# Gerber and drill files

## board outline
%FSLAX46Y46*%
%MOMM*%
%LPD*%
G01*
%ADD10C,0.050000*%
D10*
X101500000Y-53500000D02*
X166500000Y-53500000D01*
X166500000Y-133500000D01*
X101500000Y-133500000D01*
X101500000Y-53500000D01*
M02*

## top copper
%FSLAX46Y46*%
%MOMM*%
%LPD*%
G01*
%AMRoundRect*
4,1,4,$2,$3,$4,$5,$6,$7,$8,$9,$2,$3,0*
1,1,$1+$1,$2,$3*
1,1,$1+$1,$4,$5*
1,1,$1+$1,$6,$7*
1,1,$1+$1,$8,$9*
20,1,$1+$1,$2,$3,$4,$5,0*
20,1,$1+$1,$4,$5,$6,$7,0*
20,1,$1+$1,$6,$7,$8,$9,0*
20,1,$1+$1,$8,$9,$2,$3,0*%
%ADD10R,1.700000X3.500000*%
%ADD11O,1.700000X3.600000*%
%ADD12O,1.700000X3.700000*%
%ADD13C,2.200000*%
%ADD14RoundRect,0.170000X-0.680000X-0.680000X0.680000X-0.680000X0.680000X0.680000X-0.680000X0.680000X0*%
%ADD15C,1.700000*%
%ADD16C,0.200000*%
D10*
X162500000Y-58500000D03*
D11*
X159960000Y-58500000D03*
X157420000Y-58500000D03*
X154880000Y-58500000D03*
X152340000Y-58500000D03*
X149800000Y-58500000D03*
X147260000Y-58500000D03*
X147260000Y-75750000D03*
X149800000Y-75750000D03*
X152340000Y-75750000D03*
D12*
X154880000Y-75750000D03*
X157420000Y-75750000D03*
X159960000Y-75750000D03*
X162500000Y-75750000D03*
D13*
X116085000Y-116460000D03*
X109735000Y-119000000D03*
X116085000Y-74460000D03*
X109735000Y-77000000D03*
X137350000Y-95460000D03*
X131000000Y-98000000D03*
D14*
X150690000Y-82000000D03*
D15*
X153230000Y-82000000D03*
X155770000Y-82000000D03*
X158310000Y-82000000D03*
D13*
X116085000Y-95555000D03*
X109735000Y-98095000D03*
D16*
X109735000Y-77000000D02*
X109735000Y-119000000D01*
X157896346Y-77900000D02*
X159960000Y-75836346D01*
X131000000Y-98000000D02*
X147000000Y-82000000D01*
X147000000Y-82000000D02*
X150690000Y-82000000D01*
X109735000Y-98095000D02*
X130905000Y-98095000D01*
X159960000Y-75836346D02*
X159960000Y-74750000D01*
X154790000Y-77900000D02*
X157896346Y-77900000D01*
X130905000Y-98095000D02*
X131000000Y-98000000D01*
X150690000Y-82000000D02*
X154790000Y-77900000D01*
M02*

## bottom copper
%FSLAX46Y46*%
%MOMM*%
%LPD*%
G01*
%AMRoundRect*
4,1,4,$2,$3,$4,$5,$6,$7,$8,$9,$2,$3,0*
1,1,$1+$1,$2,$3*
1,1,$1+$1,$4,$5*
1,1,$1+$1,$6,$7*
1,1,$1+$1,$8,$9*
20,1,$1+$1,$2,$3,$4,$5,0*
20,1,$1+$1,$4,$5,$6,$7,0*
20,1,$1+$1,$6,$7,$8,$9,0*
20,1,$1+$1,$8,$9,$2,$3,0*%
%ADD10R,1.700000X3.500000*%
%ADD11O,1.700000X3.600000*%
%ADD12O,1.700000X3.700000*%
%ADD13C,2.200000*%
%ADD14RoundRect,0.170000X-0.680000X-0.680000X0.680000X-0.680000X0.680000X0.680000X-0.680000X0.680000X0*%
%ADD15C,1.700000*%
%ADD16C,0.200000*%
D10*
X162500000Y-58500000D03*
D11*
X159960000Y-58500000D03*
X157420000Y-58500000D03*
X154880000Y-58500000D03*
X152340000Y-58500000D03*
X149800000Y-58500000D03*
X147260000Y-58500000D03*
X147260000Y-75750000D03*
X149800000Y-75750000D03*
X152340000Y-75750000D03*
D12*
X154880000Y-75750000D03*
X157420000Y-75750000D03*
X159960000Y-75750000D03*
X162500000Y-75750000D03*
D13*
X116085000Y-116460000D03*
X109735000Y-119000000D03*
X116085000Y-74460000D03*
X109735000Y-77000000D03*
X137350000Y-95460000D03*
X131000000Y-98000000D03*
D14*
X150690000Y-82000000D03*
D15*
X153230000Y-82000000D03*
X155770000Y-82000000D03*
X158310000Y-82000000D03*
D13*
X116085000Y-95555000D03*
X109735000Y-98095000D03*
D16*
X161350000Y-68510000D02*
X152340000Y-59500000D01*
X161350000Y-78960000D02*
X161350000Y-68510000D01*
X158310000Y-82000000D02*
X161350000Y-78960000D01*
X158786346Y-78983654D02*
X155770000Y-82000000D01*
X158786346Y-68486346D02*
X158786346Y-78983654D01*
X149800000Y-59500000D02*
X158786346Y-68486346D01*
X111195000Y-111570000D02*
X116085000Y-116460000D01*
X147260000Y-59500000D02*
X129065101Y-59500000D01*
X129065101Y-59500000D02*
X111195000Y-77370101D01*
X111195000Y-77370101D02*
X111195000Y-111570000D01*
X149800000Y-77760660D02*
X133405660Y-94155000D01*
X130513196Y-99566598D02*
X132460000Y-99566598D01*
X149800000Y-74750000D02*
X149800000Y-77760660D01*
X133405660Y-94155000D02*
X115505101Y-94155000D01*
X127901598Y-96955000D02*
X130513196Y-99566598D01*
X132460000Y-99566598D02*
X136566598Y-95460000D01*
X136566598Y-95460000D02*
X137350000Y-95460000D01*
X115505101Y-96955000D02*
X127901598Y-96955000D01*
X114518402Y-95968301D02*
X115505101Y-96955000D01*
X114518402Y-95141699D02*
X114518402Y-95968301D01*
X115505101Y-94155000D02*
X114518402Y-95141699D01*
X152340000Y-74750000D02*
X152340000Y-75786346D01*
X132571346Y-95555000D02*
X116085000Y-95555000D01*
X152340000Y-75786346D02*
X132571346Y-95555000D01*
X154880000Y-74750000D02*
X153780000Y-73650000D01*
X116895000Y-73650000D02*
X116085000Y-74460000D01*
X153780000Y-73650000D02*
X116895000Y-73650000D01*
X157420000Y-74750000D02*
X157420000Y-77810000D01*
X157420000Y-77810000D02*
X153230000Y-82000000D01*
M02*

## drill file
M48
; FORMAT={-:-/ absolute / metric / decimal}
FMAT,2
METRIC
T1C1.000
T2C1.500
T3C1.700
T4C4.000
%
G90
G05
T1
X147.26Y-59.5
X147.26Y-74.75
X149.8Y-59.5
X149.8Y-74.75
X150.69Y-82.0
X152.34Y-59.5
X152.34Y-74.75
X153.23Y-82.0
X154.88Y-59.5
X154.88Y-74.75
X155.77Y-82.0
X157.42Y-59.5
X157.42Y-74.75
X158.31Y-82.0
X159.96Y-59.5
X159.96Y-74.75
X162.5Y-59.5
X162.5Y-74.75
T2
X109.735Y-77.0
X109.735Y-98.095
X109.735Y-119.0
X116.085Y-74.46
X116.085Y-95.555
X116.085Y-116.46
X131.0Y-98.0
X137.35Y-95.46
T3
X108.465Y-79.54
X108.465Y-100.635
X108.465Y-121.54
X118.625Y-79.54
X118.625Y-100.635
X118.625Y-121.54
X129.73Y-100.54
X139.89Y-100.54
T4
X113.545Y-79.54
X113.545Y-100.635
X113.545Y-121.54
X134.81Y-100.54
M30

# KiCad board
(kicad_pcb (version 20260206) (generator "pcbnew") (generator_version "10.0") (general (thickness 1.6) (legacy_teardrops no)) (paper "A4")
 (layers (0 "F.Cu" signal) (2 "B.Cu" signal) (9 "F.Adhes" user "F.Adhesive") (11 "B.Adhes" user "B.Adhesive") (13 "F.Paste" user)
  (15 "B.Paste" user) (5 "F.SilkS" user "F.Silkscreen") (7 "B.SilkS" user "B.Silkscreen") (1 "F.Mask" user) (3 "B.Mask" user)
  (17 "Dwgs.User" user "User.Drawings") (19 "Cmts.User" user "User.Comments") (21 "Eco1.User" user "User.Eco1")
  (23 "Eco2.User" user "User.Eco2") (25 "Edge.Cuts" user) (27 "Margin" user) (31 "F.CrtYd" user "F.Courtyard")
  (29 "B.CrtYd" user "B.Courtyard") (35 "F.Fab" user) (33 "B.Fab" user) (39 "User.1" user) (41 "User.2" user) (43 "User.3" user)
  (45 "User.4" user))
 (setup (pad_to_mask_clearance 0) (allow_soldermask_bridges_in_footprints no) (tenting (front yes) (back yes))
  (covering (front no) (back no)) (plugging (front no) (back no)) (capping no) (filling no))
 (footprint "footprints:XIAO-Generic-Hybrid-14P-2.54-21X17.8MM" (layer "F.Cu") (at 154.88 67.125 -90)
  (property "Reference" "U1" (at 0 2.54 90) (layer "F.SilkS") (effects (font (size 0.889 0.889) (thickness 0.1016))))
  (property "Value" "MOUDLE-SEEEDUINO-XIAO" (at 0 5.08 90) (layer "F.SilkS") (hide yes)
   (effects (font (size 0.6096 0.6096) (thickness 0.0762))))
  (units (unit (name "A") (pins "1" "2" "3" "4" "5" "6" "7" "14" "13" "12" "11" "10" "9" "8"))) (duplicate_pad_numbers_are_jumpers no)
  (pad "1" thru_hole rect (at -7.625 -7.62 270) (size 3.5 1.7) (drill 1 (offset -1 0)) (layers "*.Cu" "*.Mask") (remove_unused_layers no)
   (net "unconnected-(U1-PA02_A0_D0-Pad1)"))
  (pad "2" thru_hole oval (at -7.625 -5.08 270) (size 3.6 1.7) (drill 1 (offset -1 0)) (layers "*.Cu" "*.Mask") (remove_unused_layers no)
   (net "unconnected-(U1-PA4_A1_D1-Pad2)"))
  (pad "3" thru_hole oval (at -7.625 -2.54 270) (size 3.6 1.7) (drill 1 (offset -1 0)) (layers "*.Cu" "*.Mask") (remove_unused_layers no)
   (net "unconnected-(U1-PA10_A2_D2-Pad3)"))
  (pad "4" thru_hole oval (at -7.625 0 270) (size 3.6 1.7) (drill 1 (offset -1 0)) (layers "*.Cu" "*.Mask") (remove_unused_layers no)
   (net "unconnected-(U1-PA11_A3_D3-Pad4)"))
  (pad "5" thru_hole oval (at -7.625 2.54 270) (size 3.6 1.7) (drill 1 (offset -1 0)) (layers "*.Cu" "*.Mask") (remove_unused_layers no)
   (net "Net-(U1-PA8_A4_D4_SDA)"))
  (pad "6" thru_hole oval (at -7.625 5.08 90) (size 3.6 1.7) (drill 1 (offset 1 0)) (layers "*.Cu" "*.Mask") (remove_unused_layers no)
   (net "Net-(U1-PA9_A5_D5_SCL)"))
  (pad "7" thru_hole oval (at -7.625 7.62 270) (size 3.6 1.7) (drill 1 (offset -1 0)) (layers "*.Cu" "*.Mask") (remove_unused_layers no)
   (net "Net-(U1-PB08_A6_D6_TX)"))
  (pad "8" thru_hole oval (at 7.625 7.62 270) (size 3.6 1.7) (drill 1 (offset 1 0)) (layers "*.Cu" "*.Mask") (remove_unused_layers no)
   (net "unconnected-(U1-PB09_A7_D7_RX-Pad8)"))
  (pad "9" thru_hole oval (at 7.625 5.08 270) (size 3.6 1.7) (drill 1 (offset 1 0)) (layers "*.Cu" "*.Mask") (remove_unused_layers no)
   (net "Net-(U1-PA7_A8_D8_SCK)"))
  (pad "10" thru_hole oval (at 7.625 2.54 270) (size 3.6 1.7) (drill 1 (offset 1 0)) (layers "*.Cu" "*.Mask") (remove_unused_layers no)
   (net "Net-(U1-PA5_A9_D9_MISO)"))
  (pad "11" thru_hole oval (at 7.625 0 270) (size 3.7 1.7) (drill 1 (offset 1 0)) (layers "*.Cu" "*.Mask") (remove_unused_layers no)
   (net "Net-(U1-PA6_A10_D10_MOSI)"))
  (pad "12" thru_hole oval (at 7.625 -2.54 270) (size 3.7 1.7) (drill 1 (offset 1 0)) (layers "*.Cu" "*.Mask") (remove_unused_layers no)
   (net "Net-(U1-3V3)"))
  (pad "13" thru_hole oval (at 7.625 -5.08 270) (size 3.7 1.7) (drill 1 (offset 1 0)) (layers "*.Cu" "*.Mask") (remove_unused_layers no)
   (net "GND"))
  (pad "14" thru_hole oval (at 7.625 -7.62 270) (size 3.7 1.7) (drill 1 (offset 1 0)) (layers "*.Cu" "*.Mask") (remove_unused_layers no)
   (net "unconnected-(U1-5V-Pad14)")))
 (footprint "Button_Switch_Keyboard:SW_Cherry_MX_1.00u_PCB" (layer "F.Cu") (at 116.085 116.46)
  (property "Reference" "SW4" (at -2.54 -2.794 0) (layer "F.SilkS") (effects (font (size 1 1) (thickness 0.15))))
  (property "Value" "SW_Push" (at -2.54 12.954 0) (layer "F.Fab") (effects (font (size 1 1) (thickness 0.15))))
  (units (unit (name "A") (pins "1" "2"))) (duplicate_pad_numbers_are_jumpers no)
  (pad "" np_thru_hole circle (at -7.62 5.08) (size 1.7 1.7) (drill 1.7) (layers "*.Cu" "*.Mask"))
  (pad "" np_thru_hole circle (at -2.54 5.08) (size 4 4) (drill 4) (layers "*.Cu" "*.Mask"))
  (pad "" np_thru_hole circle (at 2.54 5.08) (size 1.7 1.7) (drill 1.7) (layers "*.Cu" "*.Mask"))
  (pad "1" thru_hole circle (at 0 0) (size 2.2 2.2) (drill 1.5) (layers "*.Cu" "*.Mask") (remove_unused_layers no)
   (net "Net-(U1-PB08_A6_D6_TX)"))
  (pad "2" thru_hole circle (at -6.35 2.54) (size 2.2 2.2) (drill 1.5) (layers "*.Cu" "*.Mask") (remove_unused_layers no) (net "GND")))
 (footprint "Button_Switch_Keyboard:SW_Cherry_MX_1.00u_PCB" (layer "F.Cu") (at 116.085 74.46)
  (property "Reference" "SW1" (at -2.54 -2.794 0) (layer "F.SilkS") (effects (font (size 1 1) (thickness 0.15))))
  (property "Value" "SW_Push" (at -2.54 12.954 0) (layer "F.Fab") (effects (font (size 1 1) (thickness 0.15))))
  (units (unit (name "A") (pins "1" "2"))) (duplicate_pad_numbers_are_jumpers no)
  (pad "" np_thru_hole circle (at -7.62 5.08) (size 1.7 1.7) (drill 1.7) (layers "*.Cu" "*.Mask"))
  (pad "" np_thru_hole circle (at -2.54 5.08) (size 4 4) (drill 4) (layers "*.Cu" "*.Mask"))
  (pad "" np_thru_hole circle (at 2.54 5.08) (size 1.7 1.7) (drill 1.7) (layers "*.Cu" "*.Mask"))
  (pad "1" thru_hole circle (at 0 0) (size 2.2 2.2) (drill 1.5) (layers "*.Cu" "*.Mask") (remove_unused_layers no)
   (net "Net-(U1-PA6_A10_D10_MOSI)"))
  (pad "2" thru_hole circle (at -6.35 2.54) (size 2.2 2.2) (drill 1.5) (layers "*.Cu" "*.Mask") (remove_unused_layers no) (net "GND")))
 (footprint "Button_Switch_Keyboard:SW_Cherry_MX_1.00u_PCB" (layer "F.Cu") (at 137.35 95.46)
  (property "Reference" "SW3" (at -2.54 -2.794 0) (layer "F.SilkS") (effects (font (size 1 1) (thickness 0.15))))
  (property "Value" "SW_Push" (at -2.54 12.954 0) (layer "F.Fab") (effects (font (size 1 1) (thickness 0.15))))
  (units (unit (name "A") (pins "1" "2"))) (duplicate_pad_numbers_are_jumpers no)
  (pad "" np_thru_hole circle (at -7.62 5.08) (size 1.7 1.7) (drill 1.7) (layers "*.Cu" "*.Mask"))
  (pad "" np_thru_hole circle (at -2.54 5.08) (size 4 4) (drill 4) (layers "*.Cu" "*.Mask"))
  (pad "" np_thru_hole circle (at 2.54 5.08) (size 1.7 1.7) (drill 1.7) (layers "*.Cu" "*.Mask"))
  (pad "1" thru_hole circle (at 0 0) (size 2.2 2.2) (drill 1.5) (layers "*.Cu" "*.Mask") (remove_unused_layers no)
   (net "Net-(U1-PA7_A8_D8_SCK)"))
  (pad "2" thru_hole circle (at -6.35 2.54) (size 2.2 2.2) (drill 1.5) (layers "*.Cu" "*.Mask") (remove_unused_layers no) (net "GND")))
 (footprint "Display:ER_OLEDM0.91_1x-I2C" (layer "F.Cu") (at 150.69 82)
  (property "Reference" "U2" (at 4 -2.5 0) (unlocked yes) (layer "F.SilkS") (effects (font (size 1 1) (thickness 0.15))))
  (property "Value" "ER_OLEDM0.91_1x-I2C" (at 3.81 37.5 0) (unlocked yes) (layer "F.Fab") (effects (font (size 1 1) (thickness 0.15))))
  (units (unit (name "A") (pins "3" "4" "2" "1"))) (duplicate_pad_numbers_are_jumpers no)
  (pad "1" thru_hole roundrect (at 0 0) (size 1.7 1.7) (drill 1) (layers "*.Cu" "*.Mask") (remove_unused_layers no) (roundrect_rratio 0.1)
   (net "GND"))
  (pad "2" thru_hole circle (at 2.54 0) (size 1.7 1.7) (drill 1) (layers "*.Cu" "*.Mask") (remove_unused_layers no) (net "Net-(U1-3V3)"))
  (pad "3" thru_hole circle (at 5.08 0) (size 1.7 1.7) (drill 1) (layers "*.Cu" "*.Mask") (remove_unused_layers no)
   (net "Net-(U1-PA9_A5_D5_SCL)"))
  (pad "4" thru_hole circle (at 7.62 0) (size 1.7 1.7) (drill 1) (layers "*.Cu" "*.Mask") (remove_unused_layers no)
   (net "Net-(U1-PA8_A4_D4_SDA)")))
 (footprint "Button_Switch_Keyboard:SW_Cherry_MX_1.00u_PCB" (layer "F.Cu") (at 116.085 95.555)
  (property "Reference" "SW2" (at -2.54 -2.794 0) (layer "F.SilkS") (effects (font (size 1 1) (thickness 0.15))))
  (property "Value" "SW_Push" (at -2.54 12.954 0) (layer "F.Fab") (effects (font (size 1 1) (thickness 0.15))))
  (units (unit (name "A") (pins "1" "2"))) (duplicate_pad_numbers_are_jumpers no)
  (pad "" np_thru_hole circle (at -7.62 5.08) (size 1.7 1.7) (drill 1.7) (layers "*.Cu" "*.Mask"))
  (pad "" np_thru_hole circle (at -2.54 5.08) (size 4 4) (drill 4) (layers "*.Cu" "*.Mask"))
  (pad "" np_thru_hole circle (at 2.54 5.08) (size 1.7 1.7) (drill 1.7) (layers "*.Cu" "*.Mask"))
  (pad "1" thru_hole circle (at 0 0) (size 2.2 2.2) (drill 1.5) (layers "*.Cu" "*.Mask") (remove_unused_layers no)
   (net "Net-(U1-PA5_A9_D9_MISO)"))
  (pad "2" thru_hole circle (at -6.35 2.54) (size 2.2 2.2) (drill 1.5) (layers "*.Cu" "*.Mask") (remove_unused_layers no) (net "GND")))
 (gr_rect (start 101.5 53.5) (end 166.5 133.5) (stroke (width 0.05) (type default)) (fill no) (layer "Edge.Cuts"))
 (segment (start 161.35 68.51) (end 152.34 59.5) (width 0.2) (layer "B.Cu") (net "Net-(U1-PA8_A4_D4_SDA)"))
 (segment (start 161.35 78.96) (end 161.35 68.51) (width 0.2) (layer "B.Cu") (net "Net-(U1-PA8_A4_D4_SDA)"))
 (segment (start 158.31 82) (end 161.35 78.96) (width 0.2) (layer "B.Cu") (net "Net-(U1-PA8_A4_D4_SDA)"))
 (segment (start 158.786346 78.983654) (end 155.77 82) (width 0.2) (layer "B.Cu") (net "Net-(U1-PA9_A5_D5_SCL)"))
 (segment (start 158.786346 68.486346) (end 158.786346 78.983654) (width 0.2) (layer "B.Cu") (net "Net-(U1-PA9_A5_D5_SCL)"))
 (segment (start 149.8 59.5) (end 158.786346 68.486346) (width 0.2) (layer "B.Cu") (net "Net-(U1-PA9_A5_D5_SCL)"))
 (segment (start 111.195 111.57) (end 116.085 116.46) (width 0.2) (layer "B.Cu") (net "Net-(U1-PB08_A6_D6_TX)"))
 (segment (start 147.26 59.5) (end 129.065101 59.5) (width 0.2) (layer "B.Cu") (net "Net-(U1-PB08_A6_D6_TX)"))
 (segment (start 129.065101 59.5) (end 111.195 77.370101) (width 0.2) (layer "B.Cu") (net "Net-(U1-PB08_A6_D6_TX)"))
 (segment (start 111.195 77.370101) (end 111.195 111.57) (width 0.2) (layer "B.Cu") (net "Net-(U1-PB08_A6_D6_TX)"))
 (segment (start 149.8 77.76066) (end 133.40566 94.155) (width 0.2) (layer "B.Cu") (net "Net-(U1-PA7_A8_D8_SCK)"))
 (segment (start 130.513196 99.566598) (end 132.46 99.566598) (width 0.2) (layer "B.Cu") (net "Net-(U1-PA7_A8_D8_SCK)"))
 (segment (start 149.8 74.75) (end 149.8 77.76066) (width 0.2) (layer "B.Cu") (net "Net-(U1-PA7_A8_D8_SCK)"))
 (segment (start 133.40566 94.155) (end 115.505101 94.155) (width 0.2) (layer "B.Cu") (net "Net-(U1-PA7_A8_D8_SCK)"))
 (segment (start 127.901598 96.955) (end 130.513196 99.566598) (width 0.2) (layer "B.Cu") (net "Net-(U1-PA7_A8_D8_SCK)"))
 (segment (start 132.46 99.566598) (end 136.566598 95.46) (width 0.2) (layer "B.Cu") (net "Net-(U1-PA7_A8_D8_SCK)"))
 (segment (start 136.566598 95.46) (end 137.35 95.46) (width 0.2) (layer "B.Cu") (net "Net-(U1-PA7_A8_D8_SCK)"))
 (segment (start 115.505101 96.955) (end 127.901598 96.955) (width 0.2) (layer "B.Cu") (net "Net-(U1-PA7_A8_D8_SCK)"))
 (segment (start 114.518402 95.968301) (end 115.505101 96.955) (width 0.2) (layer "B.Cu") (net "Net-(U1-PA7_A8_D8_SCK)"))
 (segment (start 114.518402 95.141699) (end 114.518402 95.968301) (width 0.2) (layer "B.Cu") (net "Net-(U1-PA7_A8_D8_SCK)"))
 (segment (start 115.505101 94.155) (end 114.518402 95.141699) (width 0.2) (layer "B.Cu") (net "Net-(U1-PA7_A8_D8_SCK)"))
 (segment (start 152.34 74.75) (end 152.34 75.786346) (width 0.2) (layer "B.Cu") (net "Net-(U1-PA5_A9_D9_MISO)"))
 (segment (start 132.571346 95.555) (end 116.085 95.555) (width 0.2) (layer "B.Cu") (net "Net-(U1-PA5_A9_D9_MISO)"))
 (segment (start 152.34 75.786346) (end 132.571346 95.555) (width 0.2) (layer "B.Cu") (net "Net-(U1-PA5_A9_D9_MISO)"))
 (segment (start 154.88 74.75) (end 153.78 73.65) (width 0.2) (layer "B.Cu") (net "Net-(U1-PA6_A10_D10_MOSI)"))
 (segment (start 116.895 73.65) (end 116.085 74.46) (width 0.2) (layer "B.Cu") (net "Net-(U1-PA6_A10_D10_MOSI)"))
 (segment (start 153.78 73.65) (end 116.895 73.65) (width 0.2) (layer "B.Cu") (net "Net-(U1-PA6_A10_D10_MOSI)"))
 (segment (start 157.42 74.75) (end 157.42 77.81) (width 0.2) (layer "B.Cu") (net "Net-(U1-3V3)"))
 (segment (start 157.42 77.81) (end 153.23 82) (width 0.2) (layer "B.Cu") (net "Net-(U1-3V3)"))
 (segment (start 109.735 77) (end 109.735 119) (width 0.2) (layer "F.Cu") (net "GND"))
 (segment (start 157.896346 77.9) (end 159.96 75.836346) (width 0.2) (layer "F.Cu") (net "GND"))
 (segment (start 131 98) (end 147 82) (width 0.2) (layer "F.Cu") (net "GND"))
 (segment (start 147 82) (end 150.69 82) (width 0.2) (layer "F.Cu") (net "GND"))
 (segment (start 109.735 98.095) (end 130.905 98.095) (width 0.2) (layer "F.Cu") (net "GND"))
 (segment (start 159.96 75.836346) (end 159.96 74.75) (width 0.2) (layer "F.Cu") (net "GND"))
 (segment (start 154.79 77.9) (end 157.896346 77.9) (width 0.2) (layer "F.Cu") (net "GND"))
 (segment (start 130.905 98.095) (end 131 98) (width 0.2) (layer "F.Cu") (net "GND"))
 (segment (start 150.69 82) (end 154.79 77.9) (width 0.2) (layer "F.Cu") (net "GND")))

